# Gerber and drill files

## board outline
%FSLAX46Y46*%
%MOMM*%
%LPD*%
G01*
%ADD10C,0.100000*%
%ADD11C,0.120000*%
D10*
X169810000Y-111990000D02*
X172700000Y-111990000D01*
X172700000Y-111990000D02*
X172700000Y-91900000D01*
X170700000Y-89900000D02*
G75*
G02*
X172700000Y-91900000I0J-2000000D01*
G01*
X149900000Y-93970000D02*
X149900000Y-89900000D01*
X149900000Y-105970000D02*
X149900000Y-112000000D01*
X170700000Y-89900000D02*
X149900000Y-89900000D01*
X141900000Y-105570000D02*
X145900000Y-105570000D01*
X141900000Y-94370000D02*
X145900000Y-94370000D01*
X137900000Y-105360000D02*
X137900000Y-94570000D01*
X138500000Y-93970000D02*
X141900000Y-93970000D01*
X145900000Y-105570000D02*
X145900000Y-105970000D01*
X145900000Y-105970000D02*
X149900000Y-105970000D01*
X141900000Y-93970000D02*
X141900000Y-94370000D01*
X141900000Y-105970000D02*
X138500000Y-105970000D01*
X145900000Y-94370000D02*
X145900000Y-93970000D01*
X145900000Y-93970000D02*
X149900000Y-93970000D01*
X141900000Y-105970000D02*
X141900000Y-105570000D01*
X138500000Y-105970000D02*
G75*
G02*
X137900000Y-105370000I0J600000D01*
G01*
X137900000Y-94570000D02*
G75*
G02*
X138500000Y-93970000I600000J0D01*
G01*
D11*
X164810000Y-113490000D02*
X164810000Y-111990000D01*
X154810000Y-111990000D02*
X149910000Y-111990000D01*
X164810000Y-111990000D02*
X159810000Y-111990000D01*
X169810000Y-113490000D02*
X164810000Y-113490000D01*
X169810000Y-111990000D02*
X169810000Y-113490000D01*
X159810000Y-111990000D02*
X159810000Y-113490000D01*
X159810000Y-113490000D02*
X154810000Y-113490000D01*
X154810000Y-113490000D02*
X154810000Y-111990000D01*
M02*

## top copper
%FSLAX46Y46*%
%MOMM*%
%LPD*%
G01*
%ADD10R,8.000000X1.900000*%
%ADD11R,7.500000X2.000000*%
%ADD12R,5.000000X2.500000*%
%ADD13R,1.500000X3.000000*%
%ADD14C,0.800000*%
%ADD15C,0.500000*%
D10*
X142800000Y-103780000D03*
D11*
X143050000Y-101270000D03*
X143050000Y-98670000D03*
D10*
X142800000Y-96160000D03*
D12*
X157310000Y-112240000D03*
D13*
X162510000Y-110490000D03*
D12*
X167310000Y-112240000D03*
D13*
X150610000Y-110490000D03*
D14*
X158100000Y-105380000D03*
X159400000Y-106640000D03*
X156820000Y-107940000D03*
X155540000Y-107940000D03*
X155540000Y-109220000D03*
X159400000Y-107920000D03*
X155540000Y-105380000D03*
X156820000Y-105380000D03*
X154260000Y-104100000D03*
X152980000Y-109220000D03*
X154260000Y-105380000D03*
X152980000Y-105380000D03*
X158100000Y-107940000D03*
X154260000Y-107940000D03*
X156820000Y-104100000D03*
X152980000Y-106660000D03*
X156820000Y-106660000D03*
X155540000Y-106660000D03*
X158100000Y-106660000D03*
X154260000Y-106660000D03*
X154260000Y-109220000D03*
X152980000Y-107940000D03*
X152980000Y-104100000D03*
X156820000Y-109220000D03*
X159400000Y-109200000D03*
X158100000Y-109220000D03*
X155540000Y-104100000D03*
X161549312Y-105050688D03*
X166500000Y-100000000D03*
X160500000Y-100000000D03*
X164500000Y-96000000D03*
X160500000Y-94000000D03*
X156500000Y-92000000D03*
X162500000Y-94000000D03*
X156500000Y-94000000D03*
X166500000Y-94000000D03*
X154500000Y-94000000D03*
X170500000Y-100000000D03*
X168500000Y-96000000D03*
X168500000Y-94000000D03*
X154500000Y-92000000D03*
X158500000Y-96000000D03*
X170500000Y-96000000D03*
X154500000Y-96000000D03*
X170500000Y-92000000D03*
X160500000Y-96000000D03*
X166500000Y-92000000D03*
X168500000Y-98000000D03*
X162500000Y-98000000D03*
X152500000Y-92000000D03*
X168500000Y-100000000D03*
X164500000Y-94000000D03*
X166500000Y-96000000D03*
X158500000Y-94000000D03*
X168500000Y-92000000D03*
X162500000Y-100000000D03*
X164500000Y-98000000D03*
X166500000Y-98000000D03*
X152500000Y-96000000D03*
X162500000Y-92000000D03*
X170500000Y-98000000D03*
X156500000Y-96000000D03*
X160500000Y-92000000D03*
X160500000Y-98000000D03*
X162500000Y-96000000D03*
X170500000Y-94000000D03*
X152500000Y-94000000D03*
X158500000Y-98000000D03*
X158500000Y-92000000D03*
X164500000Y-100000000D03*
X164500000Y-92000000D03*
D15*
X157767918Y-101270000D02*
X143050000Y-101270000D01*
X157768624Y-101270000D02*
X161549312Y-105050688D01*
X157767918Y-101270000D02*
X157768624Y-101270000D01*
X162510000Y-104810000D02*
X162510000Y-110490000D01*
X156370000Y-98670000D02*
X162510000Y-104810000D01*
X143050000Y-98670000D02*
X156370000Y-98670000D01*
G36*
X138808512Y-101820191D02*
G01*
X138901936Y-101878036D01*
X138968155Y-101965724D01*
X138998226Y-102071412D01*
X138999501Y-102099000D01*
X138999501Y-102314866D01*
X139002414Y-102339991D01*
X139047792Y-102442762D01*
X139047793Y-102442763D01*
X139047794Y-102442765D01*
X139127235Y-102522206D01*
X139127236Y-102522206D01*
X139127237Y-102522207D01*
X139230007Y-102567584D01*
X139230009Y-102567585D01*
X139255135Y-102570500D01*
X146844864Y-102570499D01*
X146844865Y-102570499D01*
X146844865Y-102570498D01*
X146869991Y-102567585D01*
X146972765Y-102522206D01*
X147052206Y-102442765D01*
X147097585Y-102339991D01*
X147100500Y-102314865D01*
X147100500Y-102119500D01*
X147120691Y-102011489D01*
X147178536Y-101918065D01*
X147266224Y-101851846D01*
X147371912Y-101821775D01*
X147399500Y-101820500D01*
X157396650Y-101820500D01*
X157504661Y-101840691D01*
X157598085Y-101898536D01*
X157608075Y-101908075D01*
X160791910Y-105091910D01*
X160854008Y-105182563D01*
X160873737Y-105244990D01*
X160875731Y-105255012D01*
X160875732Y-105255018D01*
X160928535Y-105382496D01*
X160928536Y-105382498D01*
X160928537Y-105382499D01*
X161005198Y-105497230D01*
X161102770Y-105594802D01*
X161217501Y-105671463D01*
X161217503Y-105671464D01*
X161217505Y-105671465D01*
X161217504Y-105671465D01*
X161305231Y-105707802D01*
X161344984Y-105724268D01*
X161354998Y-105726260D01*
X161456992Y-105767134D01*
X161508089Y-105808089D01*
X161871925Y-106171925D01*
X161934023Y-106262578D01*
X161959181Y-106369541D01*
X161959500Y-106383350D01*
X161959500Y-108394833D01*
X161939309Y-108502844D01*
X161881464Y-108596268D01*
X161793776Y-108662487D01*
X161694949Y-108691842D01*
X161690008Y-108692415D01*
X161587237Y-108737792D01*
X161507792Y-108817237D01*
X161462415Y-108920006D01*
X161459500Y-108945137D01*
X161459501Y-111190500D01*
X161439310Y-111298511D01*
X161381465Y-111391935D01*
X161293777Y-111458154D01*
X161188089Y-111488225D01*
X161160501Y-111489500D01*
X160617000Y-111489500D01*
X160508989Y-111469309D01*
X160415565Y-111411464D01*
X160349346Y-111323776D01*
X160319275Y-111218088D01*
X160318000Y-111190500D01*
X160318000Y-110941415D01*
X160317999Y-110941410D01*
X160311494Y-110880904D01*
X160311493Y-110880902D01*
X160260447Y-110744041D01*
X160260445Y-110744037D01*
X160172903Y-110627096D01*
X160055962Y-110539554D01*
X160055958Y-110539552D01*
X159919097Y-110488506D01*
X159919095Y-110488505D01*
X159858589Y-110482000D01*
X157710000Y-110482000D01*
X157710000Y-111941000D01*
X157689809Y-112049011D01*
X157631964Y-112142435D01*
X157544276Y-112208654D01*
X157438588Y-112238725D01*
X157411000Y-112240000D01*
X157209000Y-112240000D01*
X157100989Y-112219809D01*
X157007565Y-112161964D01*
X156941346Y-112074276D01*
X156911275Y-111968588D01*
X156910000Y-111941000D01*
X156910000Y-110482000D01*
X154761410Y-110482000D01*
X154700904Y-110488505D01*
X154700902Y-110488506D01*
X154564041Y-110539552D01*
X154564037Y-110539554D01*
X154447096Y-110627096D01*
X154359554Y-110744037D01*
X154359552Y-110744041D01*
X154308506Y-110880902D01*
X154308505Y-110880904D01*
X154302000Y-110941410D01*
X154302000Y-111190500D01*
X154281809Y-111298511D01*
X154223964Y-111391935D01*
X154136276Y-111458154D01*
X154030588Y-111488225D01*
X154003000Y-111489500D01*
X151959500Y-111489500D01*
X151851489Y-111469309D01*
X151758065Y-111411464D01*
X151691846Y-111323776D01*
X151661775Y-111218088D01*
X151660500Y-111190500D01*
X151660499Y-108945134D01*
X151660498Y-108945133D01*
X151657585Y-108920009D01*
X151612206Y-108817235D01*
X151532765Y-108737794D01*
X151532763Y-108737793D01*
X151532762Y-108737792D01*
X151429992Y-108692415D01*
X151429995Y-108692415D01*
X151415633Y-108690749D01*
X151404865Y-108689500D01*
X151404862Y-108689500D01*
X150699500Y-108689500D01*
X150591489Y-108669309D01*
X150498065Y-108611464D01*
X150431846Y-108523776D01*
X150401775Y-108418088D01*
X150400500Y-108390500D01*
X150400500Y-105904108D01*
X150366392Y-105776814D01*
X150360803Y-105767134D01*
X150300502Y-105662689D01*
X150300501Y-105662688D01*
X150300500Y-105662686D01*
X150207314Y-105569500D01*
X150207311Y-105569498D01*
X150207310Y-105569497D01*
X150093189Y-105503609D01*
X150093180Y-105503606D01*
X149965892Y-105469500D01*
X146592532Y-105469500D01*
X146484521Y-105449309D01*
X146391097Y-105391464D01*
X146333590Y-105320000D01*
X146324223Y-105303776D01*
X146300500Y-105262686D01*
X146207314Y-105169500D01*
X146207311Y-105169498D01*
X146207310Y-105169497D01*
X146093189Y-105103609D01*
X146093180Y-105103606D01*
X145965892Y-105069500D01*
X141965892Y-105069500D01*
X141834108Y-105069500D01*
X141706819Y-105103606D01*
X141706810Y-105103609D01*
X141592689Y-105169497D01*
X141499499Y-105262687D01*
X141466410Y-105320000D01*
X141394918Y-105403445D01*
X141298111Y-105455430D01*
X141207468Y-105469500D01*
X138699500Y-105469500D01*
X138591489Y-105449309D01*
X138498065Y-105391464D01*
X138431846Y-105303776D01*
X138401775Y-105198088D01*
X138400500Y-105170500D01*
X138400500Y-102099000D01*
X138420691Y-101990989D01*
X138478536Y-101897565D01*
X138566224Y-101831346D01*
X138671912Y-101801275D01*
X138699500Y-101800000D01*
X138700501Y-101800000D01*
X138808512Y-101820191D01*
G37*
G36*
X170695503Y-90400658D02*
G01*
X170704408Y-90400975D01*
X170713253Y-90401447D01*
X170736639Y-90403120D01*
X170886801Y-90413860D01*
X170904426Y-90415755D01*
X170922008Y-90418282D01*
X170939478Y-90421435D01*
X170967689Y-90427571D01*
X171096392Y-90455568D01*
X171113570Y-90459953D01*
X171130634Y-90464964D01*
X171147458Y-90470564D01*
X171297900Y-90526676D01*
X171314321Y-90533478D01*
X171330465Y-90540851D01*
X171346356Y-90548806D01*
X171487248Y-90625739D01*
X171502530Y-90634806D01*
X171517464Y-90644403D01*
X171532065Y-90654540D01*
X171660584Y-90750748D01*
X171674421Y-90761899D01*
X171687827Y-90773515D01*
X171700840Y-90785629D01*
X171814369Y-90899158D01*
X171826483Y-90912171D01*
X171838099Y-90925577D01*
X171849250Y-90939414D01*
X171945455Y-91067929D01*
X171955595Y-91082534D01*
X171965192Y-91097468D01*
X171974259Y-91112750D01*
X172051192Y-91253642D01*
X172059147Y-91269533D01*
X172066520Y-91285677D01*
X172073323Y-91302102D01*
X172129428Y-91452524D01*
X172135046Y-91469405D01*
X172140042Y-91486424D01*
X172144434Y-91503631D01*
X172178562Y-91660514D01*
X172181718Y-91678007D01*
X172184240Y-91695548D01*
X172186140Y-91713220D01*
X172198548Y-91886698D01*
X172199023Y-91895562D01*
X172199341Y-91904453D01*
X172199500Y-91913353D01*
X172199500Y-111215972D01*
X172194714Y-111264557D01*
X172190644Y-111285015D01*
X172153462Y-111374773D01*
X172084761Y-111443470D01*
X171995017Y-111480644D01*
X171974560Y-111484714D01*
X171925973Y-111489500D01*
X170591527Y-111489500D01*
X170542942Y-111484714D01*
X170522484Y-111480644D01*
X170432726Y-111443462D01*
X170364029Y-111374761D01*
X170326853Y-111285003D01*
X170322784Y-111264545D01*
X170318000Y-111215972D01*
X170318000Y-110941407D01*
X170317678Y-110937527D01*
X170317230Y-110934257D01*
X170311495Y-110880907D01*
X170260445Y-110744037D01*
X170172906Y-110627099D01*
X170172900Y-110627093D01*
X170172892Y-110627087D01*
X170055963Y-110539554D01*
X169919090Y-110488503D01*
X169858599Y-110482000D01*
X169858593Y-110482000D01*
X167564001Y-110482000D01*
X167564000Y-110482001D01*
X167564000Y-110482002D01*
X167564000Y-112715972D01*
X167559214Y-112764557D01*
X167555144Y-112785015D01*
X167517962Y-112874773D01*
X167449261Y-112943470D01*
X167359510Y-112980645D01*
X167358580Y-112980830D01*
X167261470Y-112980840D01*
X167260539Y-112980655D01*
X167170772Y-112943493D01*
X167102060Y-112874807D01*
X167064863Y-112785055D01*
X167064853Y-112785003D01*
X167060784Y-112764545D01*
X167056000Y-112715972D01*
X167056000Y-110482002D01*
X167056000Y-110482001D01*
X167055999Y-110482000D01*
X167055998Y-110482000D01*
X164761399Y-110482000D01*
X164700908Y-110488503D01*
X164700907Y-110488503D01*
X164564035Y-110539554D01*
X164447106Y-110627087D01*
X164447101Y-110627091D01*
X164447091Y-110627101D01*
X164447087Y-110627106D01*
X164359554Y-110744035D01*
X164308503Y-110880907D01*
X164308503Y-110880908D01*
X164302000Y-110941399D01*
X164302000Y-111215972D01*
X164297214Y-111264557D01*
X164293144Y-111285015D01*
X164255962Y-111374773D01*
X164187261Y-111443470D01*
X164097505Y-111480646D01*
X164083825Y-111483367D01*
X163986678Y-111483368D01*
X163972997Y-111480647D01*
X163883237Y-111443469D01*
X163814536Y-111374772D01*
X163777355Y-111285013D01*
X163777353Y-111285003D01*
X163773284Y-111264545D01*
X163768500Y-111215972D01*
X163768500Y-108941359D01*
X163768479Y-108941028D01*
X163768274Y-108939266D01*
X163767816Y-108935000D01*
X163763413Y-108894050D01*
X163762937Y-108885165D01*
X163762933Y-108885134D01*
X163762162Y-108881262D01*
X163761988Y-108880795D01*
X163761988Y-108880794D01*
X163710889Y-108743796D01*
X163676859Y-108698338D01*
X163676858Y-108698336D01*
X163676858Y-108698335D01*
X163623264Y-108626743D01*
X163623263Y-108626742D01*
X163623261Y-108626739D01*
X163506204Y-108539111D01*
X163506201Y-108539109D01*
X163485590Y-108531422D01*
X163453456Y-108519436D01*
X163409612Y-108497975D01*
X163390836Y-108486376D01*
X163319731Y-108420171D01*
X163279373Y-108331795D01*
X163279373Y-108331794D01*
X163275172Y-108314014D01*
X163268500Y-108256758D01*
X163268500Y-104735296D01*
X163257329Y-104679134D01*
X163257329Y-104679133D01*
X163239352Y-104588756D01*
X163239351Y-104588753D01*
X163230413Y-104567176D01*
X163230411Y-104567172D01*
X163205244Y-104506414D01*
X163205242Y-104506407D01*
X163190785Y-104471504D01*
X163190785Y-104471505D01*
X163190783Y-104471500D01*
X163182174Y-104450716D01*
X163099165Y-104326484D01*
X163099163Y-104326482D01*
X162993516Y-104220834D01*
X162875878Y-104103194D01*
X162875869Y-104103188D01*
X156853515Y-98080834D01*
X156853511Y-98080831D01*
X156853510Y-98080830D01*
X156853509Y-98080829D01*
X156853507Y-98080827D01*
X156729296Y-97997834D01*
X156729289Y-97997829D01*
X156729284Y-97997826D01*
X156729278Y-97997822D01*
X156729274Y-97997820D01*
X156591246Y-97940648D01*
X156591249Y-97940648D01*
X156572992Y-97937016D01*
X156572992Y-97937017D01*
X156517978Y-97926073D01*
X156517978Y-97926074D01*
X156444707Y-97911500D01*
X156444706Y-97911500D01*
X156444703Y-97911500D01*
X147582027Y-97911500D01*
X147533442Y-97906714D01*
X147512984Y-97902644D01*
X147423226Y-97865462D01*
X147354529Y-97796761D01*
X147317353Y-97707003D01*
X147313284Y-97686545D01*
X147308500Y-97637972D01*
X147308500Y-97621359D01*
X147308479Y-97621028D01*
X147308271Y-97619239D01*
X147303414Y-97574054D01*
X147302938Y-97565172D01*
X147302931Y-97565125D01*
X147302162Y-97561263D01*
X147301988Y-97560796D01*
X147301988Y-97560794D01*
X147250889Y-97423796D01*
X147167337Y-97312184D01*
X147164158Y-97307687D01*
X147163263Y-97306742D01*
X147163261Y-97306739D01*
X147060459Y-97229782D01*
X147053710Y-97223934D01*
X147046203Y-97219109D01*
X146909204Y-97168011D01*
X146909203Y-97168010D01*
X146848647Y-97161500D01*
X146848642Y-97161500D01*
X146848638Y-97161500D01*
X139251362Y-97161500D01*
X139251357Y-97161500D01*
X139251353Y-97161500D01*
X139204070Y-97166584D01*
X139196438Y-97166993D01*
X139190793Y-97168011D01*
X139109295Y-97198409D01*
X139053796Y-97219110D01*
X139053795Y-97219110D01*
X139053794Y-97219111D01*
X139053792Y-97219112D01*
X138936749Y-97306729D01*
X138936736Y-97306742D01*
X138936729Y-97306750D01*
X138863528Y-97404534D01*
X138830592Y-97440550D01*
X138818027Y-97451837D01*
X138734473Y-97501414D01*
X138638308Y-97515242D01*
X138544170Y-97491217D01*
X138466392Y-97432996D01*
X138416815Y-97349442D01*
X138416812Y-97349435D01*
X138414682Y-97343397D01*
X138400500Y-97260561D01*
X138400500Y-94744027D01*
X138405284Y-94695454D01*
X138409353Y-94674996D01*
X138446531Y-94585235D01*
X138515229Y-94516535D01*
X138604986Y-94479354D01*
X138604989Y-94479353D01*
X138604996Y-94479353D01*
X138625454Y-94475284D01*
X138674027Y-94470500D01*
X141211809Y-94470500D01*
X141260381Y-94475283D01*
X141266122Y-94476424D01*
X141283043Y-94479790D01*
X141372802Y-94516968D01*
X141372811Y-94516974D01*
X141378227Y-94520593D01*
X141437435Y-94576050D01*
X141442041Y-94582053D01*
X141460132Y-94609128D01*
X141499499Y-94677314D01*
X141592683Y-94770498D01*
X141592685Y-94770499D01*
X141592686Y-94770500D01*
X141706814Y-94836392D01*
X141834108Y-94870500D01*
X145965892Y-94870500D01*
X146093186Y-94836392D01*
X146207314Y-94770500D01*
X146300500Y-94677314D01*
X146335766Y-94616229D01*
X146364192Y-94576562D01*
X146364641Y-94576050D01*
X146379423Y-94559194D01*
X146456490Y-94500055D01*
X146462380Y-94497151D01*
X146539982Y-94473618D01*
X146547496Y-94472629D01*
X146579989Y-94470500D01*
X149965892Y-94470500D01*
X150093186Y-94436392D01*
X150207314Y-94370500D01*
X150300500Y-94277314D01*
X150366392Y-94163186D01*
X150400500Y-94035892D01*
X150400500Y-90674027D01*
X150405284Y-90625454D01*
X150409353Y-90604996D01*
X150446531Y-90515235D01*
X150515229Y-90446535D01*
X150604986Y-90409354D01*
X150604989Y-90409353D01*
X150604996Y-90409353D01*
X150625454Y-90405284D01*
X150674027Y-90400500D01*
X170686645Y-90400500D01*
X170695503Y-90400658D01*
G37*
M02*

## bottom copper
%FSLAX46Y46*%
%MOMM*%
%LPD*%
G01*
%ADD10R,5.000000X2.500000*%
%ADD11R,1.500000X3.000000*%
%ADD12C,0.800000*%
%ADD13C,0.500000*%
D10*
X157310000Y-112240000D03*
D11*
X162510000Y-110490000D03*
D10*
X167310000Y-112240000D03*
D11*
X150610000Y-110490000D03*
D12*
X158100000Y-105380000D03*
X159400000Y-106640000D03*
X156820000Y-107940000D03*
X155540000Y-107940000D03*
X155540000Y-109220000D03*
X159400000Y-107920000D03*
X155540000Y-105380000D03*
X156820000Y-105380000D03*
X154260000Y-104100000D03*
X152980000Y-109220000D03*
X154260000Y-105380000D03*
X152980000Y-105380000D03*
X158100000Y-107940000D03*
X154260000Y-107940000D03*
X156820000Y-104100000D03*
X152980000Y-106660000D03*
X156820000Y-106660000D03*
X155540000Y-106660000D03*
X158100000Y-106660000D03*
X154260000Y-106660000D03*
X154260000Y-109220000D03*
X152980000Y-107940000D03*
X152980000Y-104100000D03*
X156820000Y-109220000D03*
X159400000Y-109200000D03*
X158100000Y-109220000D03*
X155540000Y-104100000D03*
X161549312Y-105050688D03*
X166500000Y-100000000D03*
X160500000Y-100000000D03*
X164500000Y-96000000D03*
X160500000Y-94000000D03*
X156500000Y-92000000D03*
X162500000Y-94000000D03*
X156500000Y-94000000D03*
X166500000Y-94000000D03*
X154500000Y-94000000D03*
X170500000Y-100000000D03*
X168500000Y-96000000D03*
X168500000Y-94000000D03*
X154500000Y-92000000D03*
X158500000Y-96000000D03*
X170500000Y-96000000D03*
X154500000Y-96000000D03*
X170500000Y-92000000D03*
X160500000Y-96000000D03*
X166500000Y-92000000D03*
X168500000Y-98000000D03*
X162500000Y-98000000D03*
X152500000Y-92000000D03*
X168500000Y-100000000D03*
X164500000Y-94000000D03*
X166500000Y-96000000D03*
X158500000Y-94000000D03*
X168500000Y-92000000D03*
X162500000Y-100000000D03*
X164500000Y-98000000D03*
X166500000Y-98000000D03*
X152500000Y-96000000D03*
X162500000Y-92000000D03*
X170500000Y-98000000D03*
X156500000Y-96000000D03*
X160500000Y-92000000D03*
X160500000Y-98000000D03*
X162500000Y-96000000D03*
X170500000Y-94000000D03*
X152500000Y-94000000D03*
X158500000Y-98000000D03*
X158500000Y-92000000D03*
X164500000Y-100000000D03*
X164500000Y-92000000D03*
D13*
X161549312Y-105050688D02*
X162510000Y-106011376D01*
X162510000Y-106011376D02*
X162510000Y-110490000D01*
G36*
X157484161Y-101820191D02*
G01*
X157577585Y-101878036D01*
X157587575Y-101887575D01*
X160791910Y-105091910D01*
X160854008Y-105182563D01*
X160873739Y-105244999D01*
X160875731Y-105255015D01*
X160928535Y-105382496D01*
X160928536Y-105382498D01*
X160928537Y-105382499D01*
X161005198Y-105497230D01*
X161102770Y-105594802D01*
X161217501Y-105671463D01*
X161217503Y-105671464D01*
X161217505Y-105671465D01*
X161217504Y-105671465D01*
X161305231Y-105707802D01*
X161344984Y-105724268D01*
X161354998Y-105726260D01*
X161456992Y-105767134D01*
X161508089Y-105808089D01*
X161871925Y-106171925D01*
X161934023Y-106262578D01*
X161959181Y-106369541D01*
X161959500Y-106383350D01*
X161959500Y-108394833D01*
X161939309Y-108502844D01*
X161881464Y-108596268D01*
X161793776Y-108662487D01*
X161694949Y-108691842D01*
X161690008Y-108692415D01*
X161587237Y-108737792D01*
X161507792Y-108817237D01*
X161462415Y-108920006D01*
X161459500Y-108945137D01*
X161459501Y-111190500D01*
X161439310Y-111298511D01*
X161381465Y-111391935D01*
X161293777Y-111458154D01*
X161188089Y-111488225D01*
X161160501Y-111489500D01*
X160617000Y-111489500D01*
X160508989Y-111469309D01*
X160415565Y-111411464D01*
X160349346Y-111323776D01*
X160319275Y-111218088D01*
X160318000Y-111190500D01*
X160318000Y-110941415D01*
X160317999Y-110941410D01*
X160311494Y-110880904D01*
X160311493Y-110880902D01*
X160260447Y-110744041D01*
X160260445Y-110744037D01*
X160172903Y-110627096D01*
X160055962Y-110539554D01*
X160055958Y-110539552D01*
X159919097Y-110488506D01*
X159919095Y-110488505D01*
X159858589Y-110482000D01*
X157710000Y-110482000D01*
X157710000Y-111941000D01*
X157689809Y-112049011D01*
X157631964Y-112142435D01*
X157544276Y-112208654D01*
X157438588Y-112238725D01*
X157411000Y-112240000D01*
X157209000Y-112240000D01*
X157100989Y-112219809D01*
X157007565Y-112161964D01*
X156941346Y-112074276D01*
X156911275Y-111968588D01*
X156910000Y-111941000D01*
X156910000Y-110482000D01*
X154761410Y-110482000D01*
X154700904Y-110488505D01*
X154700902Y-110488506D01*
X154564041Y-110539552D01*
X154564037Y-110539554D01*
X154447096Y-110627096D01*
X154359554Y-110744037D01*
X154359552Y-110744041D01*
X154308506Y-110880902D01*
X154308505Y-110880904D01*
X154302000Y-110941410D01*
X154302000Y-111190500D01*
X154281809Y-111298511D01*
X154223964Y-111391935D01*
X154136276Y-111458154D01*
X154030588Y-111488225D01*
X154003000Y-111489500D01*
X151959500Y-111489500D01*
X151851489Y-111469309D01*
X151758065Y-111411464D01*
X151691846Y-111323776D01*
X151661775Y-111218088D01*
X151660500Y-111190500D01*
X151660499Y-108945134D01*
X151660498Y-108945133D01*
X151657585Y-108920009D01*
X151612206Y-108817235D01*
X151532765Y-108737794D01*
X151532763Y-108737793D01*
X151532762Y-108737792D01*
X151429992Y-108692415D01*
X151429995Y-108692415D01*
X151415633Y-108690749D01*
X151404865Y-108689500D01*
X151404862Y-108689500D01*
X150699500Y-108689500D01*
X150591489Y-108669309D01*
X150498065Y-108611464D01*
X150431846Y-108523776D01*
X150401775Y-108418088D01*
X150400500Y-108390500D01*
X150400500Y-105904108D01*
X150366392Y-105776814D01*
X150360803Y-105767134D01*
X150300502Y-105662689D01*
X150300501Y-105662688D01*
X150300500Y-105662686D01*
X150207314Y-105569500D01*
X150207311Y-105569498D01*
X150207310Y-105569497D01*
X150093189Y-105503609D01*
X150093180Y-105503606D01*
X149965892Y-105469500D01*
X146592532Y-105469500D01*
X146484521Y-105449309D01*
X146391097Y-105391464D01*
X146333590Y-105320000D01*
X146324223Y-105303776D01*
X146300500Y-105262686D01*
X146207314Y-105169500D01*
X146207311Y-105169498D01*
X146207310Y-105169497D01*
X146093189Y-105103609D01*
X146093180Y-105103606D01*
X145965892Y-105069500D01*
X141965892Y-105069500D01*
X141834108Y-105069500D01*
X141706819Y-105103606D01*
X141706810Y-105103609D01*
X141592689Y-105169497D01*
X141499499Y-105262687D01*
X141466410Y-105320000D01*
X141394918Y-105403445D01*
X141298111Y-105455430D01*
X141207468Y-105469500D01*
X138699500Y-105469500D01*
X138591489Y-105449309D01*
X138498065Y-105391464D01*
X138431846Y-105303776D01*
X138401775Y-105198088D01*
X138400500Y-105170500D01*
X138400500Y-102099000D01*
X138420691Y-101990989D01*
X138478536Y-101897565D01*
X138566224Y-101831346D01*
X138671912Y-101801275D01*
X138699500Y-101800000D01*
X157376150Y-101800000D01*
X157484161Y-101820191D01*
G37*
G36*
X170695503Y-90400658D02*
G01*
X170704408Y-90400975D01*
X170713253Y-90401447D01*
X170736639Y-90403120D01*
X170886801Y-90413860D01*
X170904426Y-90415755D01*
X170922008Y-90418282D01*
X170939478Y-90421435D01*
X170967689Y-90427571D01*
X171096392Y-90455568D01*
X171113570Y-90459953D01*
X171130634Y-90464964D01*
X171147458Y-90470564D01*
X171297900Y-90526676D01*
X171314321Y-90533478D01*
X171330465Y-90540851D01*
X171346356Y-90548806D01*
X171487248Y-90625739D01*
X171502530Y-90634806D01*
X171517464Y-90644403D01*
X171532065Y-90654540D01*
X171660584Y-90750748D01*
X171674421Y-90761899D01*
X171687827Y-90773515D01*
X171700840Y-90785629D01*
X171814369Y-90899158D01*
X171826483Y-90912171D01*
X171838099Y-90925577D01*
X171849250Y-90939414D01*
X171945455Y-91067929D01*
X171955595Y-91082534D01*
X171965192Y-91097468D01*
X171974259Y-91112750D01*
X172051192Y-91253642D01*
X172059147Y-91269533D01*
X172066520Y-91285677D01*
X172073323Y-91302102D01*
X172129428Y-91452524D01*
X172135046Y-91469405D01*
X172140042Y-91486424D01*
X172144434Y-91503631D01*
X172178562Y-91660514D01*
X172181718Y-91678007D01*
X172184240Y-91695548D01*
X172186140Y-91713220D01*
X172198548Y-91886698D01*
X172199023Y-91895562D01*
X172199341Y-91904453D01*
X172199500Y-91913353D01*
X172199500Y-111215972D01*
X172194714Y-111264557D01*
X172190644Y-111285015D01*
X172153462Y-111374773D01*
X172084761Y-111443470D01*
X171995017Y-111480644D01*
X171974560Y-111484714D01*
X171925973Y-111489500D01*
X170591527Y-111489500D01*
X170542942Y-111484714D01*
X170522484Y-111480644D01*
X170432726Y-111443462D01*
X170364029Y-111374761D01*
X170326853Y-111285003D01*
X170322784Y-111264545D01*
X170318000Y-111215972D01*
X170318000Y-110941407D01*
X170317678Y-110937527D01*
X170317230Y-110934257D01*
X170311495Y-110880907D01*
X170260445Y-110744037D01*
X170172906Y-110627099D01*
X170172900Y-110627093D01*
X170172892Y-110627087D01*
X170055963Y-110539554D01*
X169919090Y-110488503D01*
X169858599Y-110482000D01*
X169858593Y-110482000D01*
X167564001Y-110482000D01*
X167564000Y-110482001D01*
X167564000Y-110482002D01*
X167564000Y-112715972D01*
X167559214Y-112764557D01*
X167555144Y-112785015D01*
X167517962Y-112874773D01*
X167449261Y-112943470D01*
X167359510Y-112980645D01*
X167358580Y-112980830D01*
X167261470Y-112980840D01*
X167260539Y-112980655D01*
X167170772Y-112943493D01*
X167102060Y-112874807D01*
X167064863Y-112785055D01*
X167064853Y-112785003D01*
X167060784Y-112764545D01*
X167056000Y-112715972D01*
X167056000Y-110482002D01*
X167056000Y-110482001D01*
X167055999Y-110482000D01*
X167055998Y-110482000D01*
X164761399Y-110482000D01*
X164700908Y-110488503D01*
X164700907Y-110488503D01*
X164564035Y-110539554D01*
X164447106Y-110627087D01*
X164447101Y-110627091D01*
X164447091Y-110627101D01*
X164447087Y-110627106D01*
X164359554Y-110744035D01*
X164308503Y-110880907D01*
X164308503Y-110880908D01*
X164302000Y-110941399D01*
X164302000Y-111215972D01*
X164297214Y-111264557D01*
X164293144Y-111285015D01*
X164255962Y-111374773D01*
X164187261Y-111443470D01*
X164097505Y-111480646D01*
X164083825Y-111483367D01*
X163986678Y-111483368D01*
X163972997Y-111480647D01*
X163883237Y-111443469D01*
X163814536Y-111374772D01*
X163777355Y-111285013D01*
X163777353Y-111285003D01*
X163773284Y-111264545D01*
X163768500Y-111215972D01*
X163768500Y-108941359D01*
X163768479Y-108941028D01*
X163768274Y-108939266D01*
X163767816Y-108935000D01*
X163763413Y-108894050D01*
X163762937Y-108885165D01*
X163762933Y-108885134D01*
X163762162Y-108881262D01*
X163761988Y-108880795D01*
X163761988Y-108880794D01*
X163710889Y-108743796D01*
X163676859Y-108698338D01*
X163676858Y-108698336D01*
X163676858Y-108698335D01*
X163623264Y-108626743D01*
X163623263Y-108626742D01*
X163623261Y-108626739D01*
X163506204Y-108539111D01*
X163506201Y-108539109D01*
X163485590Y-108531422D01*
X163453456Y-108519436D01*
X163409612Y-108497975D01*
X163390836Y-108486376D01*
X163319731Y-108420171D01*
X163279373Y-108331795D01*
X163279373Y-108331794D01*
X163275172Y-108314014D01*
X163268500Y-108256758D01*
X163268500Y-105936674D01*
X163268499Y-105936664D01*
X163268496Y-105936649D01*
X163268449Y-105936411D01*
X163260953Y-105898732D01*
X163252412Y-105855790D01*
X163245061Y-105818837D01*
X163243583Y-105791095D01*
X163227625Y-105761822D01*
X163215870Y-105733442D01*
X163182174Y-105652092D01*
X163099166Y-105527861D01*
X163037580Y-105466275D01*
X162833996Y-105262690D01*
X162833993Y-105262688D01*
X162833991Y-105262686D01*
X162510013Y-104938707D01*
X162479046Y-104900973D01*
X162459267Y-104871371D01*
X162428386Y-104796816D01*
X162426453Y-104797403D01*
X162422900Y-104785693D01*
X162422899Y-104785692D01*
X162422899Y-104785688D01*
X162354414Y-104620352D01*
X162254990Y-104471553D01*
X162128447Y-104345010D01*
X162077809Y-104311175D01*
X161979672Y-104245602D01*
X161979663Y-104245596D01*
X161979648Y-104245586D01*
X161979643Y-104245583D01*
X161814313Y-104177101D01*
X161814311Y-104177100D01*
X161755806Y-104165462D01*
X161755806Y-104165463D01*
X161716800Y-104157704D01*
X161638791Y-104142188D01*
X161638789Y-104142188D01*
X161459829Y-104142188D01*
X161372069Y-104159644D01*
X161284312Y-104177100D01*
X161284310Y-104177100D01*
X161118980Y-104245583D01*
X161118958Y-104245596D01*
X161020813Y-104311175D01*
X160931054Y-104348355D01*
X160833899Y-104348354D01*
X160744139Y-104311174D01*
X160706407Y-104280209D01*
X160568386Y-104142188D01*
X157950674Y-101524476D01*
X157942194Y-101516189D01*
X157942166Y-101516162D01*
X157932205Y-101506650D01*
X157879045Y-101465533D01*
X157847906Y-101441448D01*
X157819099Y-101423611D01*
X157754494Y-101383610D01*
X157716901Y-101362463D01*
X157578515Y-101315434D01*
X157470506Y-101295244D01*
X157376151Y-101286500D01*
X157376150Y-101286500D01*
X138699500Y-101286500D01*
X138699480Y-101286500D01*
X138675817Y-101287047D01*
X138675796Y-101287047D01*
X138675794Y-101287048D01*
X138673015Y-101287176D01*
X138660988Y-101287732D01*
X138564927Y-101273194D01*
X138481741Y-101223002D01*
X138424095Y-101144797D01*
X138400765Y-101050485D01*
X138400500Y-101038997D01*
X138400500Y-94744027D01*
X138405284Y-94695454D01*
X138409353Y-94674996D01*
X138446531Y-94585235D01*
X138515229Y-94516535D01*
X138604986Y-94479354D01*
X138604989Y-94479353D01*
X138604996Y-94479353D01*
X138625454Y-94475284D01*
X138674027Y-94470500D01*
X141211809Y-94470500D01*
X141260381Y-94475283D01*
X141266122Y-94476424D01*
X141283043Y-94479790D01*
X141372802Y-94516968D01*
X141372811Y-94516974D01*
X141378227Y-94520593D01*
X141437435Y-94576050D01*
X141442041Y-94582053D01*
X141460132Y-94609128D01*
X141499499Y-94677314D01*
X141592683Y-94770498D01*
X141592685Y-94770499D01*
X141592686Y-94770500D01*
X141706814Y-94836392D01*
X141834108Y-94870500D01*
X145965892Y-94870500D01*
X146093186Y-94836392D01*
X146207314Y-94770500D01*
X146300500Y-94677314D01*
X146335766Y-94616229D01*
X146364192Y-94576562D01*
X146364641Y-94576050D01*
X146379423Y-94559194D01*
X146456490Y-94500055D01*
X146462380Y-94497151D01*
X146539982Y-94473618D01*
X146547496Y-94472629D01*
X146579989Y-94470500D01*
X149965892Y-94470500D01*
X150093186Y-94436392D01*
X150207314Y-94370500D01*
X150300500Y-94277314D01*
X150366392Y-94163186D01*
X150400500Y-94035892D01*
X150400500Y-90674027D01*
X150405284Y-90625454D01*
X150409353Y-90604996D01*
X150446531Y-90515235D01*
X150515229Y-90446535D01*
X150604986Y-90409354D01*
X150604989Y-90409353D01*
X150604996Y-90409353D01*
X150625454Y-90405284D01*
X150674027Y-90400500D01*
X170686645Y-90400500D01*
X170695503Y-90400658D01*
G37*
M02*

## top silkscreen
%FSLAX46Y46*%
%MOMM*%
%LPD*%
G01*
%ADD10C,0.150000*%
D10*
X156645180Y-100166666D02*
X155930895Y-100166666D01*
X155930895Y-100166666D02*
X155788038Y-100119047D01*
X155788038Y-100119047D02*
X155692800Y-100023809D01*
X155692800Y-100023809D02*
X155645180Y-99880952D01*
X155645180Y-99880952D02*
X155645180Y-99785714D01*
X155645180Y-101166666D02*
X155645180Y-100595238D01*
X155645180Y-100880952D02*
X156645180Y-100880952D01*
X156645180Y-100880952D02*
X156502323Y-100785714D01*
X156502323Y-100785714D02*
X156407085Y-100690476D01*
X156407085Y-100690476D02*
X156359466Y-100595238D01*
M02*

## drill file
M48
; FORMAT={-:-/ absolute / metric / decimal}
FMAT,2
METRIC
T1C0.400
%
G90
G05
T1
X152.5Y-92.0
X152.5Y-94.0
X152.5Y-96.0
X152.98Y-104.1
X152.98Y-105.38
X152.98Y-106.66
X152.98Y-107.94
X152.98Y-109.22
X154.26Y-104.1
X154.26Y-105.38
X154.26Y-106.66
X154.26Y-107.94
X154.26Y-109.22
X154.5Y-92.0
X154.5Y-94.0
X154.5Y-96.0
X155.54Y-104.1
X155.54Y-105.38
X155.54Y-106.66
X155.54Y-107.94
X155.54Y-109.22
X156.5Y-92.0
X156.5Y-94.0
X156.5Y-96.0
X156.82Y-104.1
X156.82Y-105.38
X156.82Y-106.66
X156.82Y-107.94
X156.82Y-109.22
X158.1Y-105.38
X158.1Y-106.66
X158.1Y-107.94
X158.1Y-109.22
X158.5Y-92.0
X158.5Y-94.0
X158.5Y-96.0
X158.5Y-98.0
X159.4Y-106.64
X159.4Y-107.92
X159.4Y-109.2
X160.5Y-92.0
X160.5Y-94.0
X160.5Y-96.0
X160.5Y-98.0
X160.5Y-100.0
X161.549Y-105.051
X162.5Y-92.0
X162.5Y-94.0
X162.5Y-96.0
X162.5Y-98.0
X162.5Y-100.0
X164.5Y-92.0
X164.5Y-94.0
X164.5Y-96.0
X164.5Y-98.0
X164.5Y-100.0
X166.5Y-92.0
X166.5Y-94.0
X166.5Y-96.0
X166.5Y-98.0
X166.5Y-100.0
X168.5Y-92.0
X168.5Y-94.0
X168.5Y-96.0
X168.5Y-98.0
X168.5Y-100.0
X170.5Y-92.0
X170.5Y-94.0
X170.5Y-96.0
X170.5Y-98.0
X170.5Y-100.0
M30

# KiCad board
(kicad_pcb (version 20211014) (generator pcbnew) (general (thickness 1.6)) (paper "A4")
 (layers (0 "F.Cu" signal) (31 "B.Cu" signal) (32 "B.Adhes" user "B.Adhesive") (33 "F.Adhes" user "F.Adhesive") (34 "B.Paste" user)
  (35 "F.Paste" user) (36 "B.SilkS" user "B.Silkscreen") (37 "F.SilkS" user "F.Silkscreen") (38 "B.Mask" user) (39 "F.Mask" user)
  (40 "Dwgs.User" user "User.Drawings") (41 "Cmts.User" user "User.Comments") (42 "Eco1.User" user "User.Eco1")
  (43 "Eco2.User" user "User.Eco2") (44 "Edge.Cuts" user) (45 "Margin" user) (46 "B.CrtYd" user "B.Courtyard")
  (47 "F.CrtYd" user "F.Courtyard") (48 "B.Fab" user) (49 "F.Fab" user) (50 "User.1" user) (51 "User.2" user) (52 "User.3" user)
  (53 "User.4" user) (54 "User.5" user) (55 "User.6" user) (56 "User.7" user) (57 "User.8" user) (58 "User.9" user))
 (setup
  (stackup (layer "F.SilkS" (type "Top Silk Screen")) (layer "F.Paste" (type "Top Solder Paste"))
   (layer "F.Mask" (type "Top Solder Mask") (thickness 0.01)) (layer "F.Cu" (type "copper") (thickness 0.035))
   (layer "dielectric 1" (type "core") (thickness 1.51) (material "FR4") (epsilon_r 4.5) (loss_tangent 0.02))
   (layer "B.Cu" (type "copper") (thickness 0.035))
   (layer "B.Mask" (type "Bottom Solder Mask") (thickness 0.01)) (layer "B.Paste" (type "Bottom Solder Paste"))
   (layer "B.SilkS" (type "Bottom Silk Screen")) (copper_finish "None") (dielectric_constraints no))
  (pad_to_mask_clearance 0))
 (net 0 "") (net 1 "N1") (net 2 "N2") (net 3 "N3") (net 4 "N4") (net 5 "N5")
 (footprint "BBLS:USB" (layer "F.Cu") (at 150 100 -90)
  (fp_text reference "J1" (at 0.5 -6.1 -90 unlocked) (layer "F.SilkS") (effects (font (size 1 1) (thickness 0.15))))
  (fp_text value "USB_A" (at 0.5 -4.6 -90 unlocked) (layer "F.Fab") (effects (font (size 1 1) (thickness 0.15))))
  (fp_line (start 5.57 8.1) (end 5.57 4.1) (layer "Edge.Cuts") (width 0.1))
  (fp_line (start -5.63 8.1) (end -5.63 4.1) (layer "Edge.Cuts") (width 0.1))
  (fp_line (start 5.36 12.1) (end -5.43 12.1) (layer "Edge.Cuts") (width 0.1))
  (fp_line (start -6.03 11.5) (end -6.03 8.1) (layer "Edge.Cuts") (width 0.1))
  (fp_line (start 5.57 4.1) (end 5.97 4.1) (layer "Edge.Cuts") (width 0.1))
  (fp_line (start 5.97 4.1) (end 5.97 0.1) (layer "Edge.Cuts") (width 0.1))
  (fp_line (start -6.03 8.1) (end -5.63 8.1) (layer "Edge.Cuts") (width 0.1))
  (fp_line (start 5.97 8.1) (end 5.97 11.5) (layer "Edge.Cuts") (width 0.1))
  (fp_line (start -5.63 4.1) (end -6.03 4.1) (layer "Edge.Cuts") (width 0.1))
  (fp_line (start -6.03 4.1) (end -6.03 0.1) (layer "Edge.Cuts") (width 0.1))
  (fp_line (start 5.97 8.1) (end 5.57 8.1) (layer "Edge.Cuts") (width 0.1))
  (fp_arc (start 5.97 11.5) (mid 5.794264 11.924264) (end 5.37 12.1) (layer "Edge.Cuts") (width 0.1))
  (fp_arc (start -5.43 12.1) (mid -5.854264 11.924264) (end -6.03 11.5) (layer "Edge.Cuts") (width 0.1))
  (pad "1" connect rect (at 3.78 7.2 270) (size 1.9 8) (layers "F.Cu" "F.Mask") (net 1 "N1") (zone_connect 2))
  (pad "2" connect rect (at 1.27 6.95 270) (size 2 7.5) (layers "F.Cu" "F.Mask") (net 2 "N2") (zone_connect 2))
  (pad "3" connect rect (at -1.33 6.95 270) (size 2 7.5) (layers "F.Cu" "F.Mask") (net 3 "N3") (zone_connect 2))
  (pad "4" connect rect (at -3.84 7.2 270) (size 1.9 8) (layers "F.Cu" "F.Mask") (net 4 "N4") (zone_connect 2)))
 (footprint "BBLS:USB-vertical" (layer "B.Cu") (at 162.31 110.99 180)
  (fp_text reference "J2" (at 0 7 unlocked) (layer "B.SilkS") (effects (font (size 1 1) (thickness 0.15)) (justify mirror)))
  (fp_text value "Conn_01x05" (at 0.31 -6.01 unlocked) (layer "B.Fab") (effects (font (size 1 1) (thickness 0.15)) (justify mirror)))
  (fp_line (start -2.5 -2.5) (end -2.5 -1) (layer "Edge.Cuts") (width 0.12))
  (fp_line (start 7.5 -1) (end 12.4 -1) (layer "Edge.Cuts") (width 0.12))
  (fp_line (start -2.5 -1) (end 2.5 -1) (layer "Edge.Cuts") (width 0.12))
  (fp_line (start -7.5 -2.5) (end -2.5 -2.5) (layer "Edge.Cuts") (width 0.12))
  (fp_line (start -7.5 -1) (end -7.5 -2.5) (layer "Edge.Cuts") (width 0.12))
  (fp_line (start 2.5 -1) (end 2.5 -2.5) (layer "Edge.Cuts") (width 0.12))
  (fp_line (start 2.5 -2.5) (end 7.5 -2.5) (layer "Edge.Cuts") (width 0.12))
  (fp_line (start 7.5 -2.5) (end 7.5 -1) (layer "Edge.Cuts") (width 0.12))
  (pad "1" smd rect (at 5 -1.25 270) (size 2.5 5) (layers "F.Cu" "F.Paste" "F.Mask") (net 1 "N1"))
  (pad "1" smd rect (at 5 -1.25 90) (size 2.5 5) (layers "B.Cu" "B.Paste" "B.Mask") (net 1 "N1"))
  (pad "2" smd rect (at -0.2 0.5 180) (size 1.5 3) (layers "F.Cu" "F.Paste" "F.Mask") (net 3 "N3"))
  (pad "3" smd rect (at -0.2 0.5) (size 1.5 3) (layers "B.Cu" "B.Paste" "B.Mask") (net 2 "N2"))
  (pad "4" smd rect (at -5 -1.25 270) (size 2.5 5) (layers "F.Cu" "F.Paste" "F.Mask") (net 4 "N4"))
  (pad "4" smd rect (at -5 -1.25 90) (size 2.5 5) (layers "B.Cu" "B.Paste" "B.Mask") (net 4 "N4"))
  (pad "5" smd rect (at 11.7 0.5) (size 1.5 3) (layers "F.Cu" "F.Paste" "F.Mask") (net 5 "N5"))
  (pad "5" smd rect (at 11.7 0.5) (size 1.5 3) (layers "B.Cu" "B.Paste" "B.Mask") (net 5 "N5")))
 (gr_line (start 169.81 111.99) (end 172.7 111.99) (layer "Edge.Cuts") (width 0.1))
 (gr_line (start 172.7 111.99) (end 172.7 91.9) (layer "Edge.Cuts") (width 0.1))
 (gr_arc (start 170.7 89.9) (mid 172.114214 90.485786) (end 172.7 91.9) (layer "Edge.Cuts") (width 0.1))
 (gr_line (start 149.9 93.97) (end 149.9 89.9) (layer "Edge.Cuts") (width 0.1))
 (gr_line (start 149.9 105.97) (end 149.9 112) (layer "Edge.Cuts") (width 0.1))
 (gr_line (start 170.7 89.9) (end 149.9 89.9) (layer "Edge.Cuts") (width 0.1))
 (via (at 158.1 105.38) (size 0.8) (drill 0.4) (layers "F.Cu" "B.Cu") (free) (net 1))
 (via (at 159.4 106.64) (size 0.8) (drill 0.4) (layers "F.Cu" "B.Cu") (free) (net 1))
 (via (at 156.82 107.94) (size 0.8) (drill 0.4) (layers "F.Cu" "B.Cu") (free) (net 1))
 (via (at 155.54 107.94) (size 0.8) (drill 0.4) (layers "F.Cu" "B.Cu") (free) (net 1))
 (via (at 155.54 109.22) (size 0.8) (drill 0.4) (layers "F.Cu" "B.Cu") (free) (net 1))
 (via (at 159.4 107.92) (size 0.8) (drill 0.4) (layers "F.Cu" "B.Cu") (free) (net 1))
 (via (at 155.54 105.38) (size 0.8) (drill 0.4) (layers "F.Cu" "B.Cu") (free) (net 1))
 (via (at 156.82 105.38) (size 0.8) (drill 0.4) (layers "F.Cu" "B.Cu") (free) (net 1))
 (via (at 154.26 104.1) (size 0.8) (drill 0.4) (layers "F.Cu" "B.Cu") (free) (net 1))
 (via (at 152.98 109.22) (size 0.8) (drill 0.4) (layers "F.Cu" "B.Cu") (free) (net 1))
 (via (at 154.26 105.38) (size 0.8) (drill 0.4) (layers "F.Cu" "B.Cu") (free) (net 1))
 (via (at 152.98 105.38) (size 0.8) (drill 0.4) (layers "F.Cu" "B.Cu") (free) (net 1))
 (via (at 158.1 107.94) (size 0.8) (drill 0.4) (layers "F.Cu" "B.Cu") (free) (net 1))
 (via (at 154.26 107.94) (size 0.8) (drill 0.4) (layers "F.Cu" "B.Cu") (free) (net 1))
 (via (at 156.82 104.1) (size 0.8) (drill 0.4) (layers "F.Cu" "B.Cu") (free) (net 1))
 (via (at 152.98 106.66) (size 0.8) (drill 0.4) (layers "F.Cu" "B.Cu") (free) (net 1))
 (via (at 156.82 106.66) (size 0.8) (drill 0.4) (layers "F.Cu" "B.Cu") (free) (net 1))
 (via (at 155.54 106.66) (size 0.8) (drill 0.4) (layers "F.Cu" "B.Cu") (free) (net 1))
 (via (at 158.1 106.66) (size 0.8) (drill 0.4) (layers "F.Cu" "B.Cu") (free) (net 1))
 (via (at 154.26 106.66) (size 0.8) (drill 0.4) (layers "F.Cu" "B.Cu") (free) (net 1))
 (via (at 154.26 109.22) (size 0.8) (drill 0.4) (layers "F.Cu" "B.Cu") (free) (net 1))
 (via (at 152.98 107.94) (size 0.8) (drill 0.4) (layers "F.Cu" "B.Cu") (free) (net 1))
 (via (at 152.98 104.1) (size 0.8) (drill 0.4) (layers "F.Cu" "B.Cu") (free) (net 1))
 (via (at 156.82 109.22) (size 0.8) (drill 0.4) (layers "F.Cu" "B.Cu") (free) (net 1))
 (via (at 159.4 109.2) (size 0.8) (drill 0.4) (layers "F.Cu" "B.Cu") (free) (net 1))
 (via (at 158.1 109.22) (size 0.8) (drill 0.4) (layers "F.Cu" "B.Cu") (free) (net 1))
 (via (at 155.54 104.1) (size 0.8) (drill 0.4) (layers "F.Cu" "B.Cu") (free) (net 1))
 (segment (start 157.767918 101.27) (end 143.05 101.27) (width 0.5) (layer "F.Cu") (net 2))
 (segment (start 157.768624 101.27) (end 161.549312 105.050688) (width 0.5) (layer "F.Cu") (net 2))
 (segment (start 157.767918 101.27) (end 157.768624 101.27) (width 0.5) (layer "F.Cu") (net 2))
 (via (at 161.549312 105.050688) (size 0.8) (drill 0.4) (layers "F.Cu" "B.Cu") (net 2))
 (segment (start 161.549312 105.050688) (end 162.51 106.011376) (width 0.5) (layer "B.Cu") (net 2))
 (segment (start 162.51 106.011376) (end 162.51 110.49) (width 0.5) (layer "B.Cu") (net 2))
 (segment (start 162.51 104.81) (end 162.51 110.49) (width 0.5) (layer "F.Cu") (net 3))
 (segment (start 156.37 98.67) (end 162.51 104.81) (width 0.5) (layer "F.Cu") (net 3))
 (segment (start 143.05 98.67) (end 156.37 98.67) (width 0.5) (layer "F.Cu") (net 3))
 (via (at 166.5 100) (size 0.8) (drill 0.4) (layers "F.Cu" "B.Cu") (free) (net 4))
 (via (at 160.5 100) (size 0.8) (drill 0.4) (layers "F.Cu" "B.Cu") (free) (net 4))
 (via (at 164.5 96) (size 0.8) (drill 0.4) (layers "F.Cu" "B.Cu") (free) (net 4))
 (via (at 160.5 94) (size 0.8) (drill 0.4) (layers "F.Cu" "B.Cu") (free) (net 4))
 (via (at 156.5 92) (size 0.8) (drill 0.4) (layers "F.Cu" "B.Cu") (free) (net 4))
 (via (at 162.5 94) (size 0.8) (drill 0.4) (layers "F.Cu" "B.Cu") (free) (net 4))
 (via (at 156.5 94) (size 0.8) (drill 0.4) (layers "F.Cu" "B.Cu") (free) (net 4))
 (via (at 166.5 94) (size 0.8) (drill 0.4) (layers "F.Cu" "B.Cu") (free) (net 4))
 (via (at 154.5 94) (size 0.8) (drill 0.4) (layers "F.Cu" "B.Cu") (free) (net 4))
 (via (at 170.5 100) (size 0.8) (drill 0.4) (layers "F.Cu" "B.Cu") (free) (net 4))
 (via (at 168.5 96) (size 0.8) (drill 0.4) (layers "F.Cu" "B.Cu") (free) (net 4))
 (via (at 168.5 94) (size 0.8) (drill 0.4) (layers "F.Cu" "B.Cu") (free) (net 4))
 (via (at 154.5 92) (size 0.8) (drill 0.4) (layers "F.Cu" "B.Cu") (free) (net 4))
 (via (at 158.5 96) (size 0.8) (drill 0.4) (layers "F.Cu" "B.Cu") (free) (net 4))
 (via (at 170.5 96) (size 0.8) (drill 0.4) (layers "F.Cu" "B.Cu") (free) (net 4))
 (via (at 154.5 96) (size 0.8) (drill 0.4) (layers "F.Cu" "B.Cu") (free) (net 4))
 (via (at 170.5 92) (size 0.8) (drill 0.4) (layers "F.Cu" "B.Cu") (free) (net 4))
 (via (at 160.5 96) (size 0.8) (drill 0.4) (layers "F.Cu" "B.Cu") (free) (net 4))
 (via (at 166.5 92) (size 0.8) (drill 0.4) (layers "F.Cu" "B.Cu") (free) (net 4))
 (via (at 168.5 98) (size 0.8) (drill 0.4) (layers "F.Cu" "B.Cu") (free) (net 4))
 (via (at 162.5 98) (size 0.8) (drill 0.4) (layers "F.Cu" "B.Cu") (free) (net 4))
 (via (at 152.5 92) (size 0.8) (drill 0.4) (layers "F.Cu" "B.Cu") (free) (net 4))
 (via (at 168.5 100) (size 0.8) (drill 0.4) (layers "F.Cu" "B.Cu") (free) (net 4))
 (via (at 164.5 94) (size 0.8) (drill 0.4) (layers "F.Cu" "B.Cu") (free) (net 4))
 (via (at 166.5 96) (size 0.8) (drill 0.4) (layers "F.Cu" "B.Cu") (free) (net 4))
 (via (at 158.5 94) (size 0.8) (drill 0.4) (layers "F.Cu" "B.Cu") (free) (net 4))
 (via (at 168.5 92) (size 0.8) (drill 0.4) (layers "F.Cu" "B.Cu") (free) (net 4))
 (via (at 162.5 100) (size 0.8) (drill 0.4) (layers "F.Cu" "B.Cu") (free) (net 4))
 (via (at 164.5 98) (size 0.8) (drill 0.4) (layers "F.Cu" "B.Cu") (free) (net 4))
 (via (at 166.5 98) (size 0.8) (drill 0.4) (layers "F.Cu" "B.Cu") (free) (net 4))
 (via (at 152.5 96) (size 0.8) (drill 0.4) (layers "F.Cu" "B.Cu") (free) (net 4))
 (via (at 162.5 92) (size 0.8) (drill 0.4) (layers "F.Cu" "B.Cu") (free) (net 4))
 (via (at 170.5 98) (size 0.8) (drill 0.4) (layers "F.Cu" "B.Cu") (free) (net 4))
 (via (at 156.5 96) (size 0.8) (drill 0.4) (layers "F.Cu" "B.Cu") (free) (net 4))
 (via (at 160.5 92) (size 0.8) (drill 0.4) (layers "F.Cu" "B.Cu") (free) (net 4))
 (via (at 160.5 98) (size 0.8) (drill 0.4) (layers "F.Cu" "B.Cu") (free) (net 4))
 (via (at 162.5 96) (size 0.8) (drill 0.4) (layers "F.Cu" "B.Cu") (free) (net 4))
 (via (at 170.5 94) (size 0.8) (drill 0.4) (layers "F.Cu" "B.Cu") (free) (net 4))
 (via (at 152.5 94) (size 0.8) (drill 0.4) (layers "F.Cu" "B.Cu") (free) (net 4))
 (via (at 158.5 98) (size 0.8) (drill 0.4) (layers "F.Cu" "B.Cu") (free) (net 4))
 (via (at 158.5 92) (size 0.8) (drill 0.4) (layers "F.Cu" "B.Cu") (free) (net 4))
 (via (at 164.5 100) (size 0.8) (drill 0.4) (layers "F.Cu" "B.Cu") (free) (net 4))
 (via (at 164.5 92) (size 0.8) (drill 0.4) (layers "F.Cu" "B.Cu") (free) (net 4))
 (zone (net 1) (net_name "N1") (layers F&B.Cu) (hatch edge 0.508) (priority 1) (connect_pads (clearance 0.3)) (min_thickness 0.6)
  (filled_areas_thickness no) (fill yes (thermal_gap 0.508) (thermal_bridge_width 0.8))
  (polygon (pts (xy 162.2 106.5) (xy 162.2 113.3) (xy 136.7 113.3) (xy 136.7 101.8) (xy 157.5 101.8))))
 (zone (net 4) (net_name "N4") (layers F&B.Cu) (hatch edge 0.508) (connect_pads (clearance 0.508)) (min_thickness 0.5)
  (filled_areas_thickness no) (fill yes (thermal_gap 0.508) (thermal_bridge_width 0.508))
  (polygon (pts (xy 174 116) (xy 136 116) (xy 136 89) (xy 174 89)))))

